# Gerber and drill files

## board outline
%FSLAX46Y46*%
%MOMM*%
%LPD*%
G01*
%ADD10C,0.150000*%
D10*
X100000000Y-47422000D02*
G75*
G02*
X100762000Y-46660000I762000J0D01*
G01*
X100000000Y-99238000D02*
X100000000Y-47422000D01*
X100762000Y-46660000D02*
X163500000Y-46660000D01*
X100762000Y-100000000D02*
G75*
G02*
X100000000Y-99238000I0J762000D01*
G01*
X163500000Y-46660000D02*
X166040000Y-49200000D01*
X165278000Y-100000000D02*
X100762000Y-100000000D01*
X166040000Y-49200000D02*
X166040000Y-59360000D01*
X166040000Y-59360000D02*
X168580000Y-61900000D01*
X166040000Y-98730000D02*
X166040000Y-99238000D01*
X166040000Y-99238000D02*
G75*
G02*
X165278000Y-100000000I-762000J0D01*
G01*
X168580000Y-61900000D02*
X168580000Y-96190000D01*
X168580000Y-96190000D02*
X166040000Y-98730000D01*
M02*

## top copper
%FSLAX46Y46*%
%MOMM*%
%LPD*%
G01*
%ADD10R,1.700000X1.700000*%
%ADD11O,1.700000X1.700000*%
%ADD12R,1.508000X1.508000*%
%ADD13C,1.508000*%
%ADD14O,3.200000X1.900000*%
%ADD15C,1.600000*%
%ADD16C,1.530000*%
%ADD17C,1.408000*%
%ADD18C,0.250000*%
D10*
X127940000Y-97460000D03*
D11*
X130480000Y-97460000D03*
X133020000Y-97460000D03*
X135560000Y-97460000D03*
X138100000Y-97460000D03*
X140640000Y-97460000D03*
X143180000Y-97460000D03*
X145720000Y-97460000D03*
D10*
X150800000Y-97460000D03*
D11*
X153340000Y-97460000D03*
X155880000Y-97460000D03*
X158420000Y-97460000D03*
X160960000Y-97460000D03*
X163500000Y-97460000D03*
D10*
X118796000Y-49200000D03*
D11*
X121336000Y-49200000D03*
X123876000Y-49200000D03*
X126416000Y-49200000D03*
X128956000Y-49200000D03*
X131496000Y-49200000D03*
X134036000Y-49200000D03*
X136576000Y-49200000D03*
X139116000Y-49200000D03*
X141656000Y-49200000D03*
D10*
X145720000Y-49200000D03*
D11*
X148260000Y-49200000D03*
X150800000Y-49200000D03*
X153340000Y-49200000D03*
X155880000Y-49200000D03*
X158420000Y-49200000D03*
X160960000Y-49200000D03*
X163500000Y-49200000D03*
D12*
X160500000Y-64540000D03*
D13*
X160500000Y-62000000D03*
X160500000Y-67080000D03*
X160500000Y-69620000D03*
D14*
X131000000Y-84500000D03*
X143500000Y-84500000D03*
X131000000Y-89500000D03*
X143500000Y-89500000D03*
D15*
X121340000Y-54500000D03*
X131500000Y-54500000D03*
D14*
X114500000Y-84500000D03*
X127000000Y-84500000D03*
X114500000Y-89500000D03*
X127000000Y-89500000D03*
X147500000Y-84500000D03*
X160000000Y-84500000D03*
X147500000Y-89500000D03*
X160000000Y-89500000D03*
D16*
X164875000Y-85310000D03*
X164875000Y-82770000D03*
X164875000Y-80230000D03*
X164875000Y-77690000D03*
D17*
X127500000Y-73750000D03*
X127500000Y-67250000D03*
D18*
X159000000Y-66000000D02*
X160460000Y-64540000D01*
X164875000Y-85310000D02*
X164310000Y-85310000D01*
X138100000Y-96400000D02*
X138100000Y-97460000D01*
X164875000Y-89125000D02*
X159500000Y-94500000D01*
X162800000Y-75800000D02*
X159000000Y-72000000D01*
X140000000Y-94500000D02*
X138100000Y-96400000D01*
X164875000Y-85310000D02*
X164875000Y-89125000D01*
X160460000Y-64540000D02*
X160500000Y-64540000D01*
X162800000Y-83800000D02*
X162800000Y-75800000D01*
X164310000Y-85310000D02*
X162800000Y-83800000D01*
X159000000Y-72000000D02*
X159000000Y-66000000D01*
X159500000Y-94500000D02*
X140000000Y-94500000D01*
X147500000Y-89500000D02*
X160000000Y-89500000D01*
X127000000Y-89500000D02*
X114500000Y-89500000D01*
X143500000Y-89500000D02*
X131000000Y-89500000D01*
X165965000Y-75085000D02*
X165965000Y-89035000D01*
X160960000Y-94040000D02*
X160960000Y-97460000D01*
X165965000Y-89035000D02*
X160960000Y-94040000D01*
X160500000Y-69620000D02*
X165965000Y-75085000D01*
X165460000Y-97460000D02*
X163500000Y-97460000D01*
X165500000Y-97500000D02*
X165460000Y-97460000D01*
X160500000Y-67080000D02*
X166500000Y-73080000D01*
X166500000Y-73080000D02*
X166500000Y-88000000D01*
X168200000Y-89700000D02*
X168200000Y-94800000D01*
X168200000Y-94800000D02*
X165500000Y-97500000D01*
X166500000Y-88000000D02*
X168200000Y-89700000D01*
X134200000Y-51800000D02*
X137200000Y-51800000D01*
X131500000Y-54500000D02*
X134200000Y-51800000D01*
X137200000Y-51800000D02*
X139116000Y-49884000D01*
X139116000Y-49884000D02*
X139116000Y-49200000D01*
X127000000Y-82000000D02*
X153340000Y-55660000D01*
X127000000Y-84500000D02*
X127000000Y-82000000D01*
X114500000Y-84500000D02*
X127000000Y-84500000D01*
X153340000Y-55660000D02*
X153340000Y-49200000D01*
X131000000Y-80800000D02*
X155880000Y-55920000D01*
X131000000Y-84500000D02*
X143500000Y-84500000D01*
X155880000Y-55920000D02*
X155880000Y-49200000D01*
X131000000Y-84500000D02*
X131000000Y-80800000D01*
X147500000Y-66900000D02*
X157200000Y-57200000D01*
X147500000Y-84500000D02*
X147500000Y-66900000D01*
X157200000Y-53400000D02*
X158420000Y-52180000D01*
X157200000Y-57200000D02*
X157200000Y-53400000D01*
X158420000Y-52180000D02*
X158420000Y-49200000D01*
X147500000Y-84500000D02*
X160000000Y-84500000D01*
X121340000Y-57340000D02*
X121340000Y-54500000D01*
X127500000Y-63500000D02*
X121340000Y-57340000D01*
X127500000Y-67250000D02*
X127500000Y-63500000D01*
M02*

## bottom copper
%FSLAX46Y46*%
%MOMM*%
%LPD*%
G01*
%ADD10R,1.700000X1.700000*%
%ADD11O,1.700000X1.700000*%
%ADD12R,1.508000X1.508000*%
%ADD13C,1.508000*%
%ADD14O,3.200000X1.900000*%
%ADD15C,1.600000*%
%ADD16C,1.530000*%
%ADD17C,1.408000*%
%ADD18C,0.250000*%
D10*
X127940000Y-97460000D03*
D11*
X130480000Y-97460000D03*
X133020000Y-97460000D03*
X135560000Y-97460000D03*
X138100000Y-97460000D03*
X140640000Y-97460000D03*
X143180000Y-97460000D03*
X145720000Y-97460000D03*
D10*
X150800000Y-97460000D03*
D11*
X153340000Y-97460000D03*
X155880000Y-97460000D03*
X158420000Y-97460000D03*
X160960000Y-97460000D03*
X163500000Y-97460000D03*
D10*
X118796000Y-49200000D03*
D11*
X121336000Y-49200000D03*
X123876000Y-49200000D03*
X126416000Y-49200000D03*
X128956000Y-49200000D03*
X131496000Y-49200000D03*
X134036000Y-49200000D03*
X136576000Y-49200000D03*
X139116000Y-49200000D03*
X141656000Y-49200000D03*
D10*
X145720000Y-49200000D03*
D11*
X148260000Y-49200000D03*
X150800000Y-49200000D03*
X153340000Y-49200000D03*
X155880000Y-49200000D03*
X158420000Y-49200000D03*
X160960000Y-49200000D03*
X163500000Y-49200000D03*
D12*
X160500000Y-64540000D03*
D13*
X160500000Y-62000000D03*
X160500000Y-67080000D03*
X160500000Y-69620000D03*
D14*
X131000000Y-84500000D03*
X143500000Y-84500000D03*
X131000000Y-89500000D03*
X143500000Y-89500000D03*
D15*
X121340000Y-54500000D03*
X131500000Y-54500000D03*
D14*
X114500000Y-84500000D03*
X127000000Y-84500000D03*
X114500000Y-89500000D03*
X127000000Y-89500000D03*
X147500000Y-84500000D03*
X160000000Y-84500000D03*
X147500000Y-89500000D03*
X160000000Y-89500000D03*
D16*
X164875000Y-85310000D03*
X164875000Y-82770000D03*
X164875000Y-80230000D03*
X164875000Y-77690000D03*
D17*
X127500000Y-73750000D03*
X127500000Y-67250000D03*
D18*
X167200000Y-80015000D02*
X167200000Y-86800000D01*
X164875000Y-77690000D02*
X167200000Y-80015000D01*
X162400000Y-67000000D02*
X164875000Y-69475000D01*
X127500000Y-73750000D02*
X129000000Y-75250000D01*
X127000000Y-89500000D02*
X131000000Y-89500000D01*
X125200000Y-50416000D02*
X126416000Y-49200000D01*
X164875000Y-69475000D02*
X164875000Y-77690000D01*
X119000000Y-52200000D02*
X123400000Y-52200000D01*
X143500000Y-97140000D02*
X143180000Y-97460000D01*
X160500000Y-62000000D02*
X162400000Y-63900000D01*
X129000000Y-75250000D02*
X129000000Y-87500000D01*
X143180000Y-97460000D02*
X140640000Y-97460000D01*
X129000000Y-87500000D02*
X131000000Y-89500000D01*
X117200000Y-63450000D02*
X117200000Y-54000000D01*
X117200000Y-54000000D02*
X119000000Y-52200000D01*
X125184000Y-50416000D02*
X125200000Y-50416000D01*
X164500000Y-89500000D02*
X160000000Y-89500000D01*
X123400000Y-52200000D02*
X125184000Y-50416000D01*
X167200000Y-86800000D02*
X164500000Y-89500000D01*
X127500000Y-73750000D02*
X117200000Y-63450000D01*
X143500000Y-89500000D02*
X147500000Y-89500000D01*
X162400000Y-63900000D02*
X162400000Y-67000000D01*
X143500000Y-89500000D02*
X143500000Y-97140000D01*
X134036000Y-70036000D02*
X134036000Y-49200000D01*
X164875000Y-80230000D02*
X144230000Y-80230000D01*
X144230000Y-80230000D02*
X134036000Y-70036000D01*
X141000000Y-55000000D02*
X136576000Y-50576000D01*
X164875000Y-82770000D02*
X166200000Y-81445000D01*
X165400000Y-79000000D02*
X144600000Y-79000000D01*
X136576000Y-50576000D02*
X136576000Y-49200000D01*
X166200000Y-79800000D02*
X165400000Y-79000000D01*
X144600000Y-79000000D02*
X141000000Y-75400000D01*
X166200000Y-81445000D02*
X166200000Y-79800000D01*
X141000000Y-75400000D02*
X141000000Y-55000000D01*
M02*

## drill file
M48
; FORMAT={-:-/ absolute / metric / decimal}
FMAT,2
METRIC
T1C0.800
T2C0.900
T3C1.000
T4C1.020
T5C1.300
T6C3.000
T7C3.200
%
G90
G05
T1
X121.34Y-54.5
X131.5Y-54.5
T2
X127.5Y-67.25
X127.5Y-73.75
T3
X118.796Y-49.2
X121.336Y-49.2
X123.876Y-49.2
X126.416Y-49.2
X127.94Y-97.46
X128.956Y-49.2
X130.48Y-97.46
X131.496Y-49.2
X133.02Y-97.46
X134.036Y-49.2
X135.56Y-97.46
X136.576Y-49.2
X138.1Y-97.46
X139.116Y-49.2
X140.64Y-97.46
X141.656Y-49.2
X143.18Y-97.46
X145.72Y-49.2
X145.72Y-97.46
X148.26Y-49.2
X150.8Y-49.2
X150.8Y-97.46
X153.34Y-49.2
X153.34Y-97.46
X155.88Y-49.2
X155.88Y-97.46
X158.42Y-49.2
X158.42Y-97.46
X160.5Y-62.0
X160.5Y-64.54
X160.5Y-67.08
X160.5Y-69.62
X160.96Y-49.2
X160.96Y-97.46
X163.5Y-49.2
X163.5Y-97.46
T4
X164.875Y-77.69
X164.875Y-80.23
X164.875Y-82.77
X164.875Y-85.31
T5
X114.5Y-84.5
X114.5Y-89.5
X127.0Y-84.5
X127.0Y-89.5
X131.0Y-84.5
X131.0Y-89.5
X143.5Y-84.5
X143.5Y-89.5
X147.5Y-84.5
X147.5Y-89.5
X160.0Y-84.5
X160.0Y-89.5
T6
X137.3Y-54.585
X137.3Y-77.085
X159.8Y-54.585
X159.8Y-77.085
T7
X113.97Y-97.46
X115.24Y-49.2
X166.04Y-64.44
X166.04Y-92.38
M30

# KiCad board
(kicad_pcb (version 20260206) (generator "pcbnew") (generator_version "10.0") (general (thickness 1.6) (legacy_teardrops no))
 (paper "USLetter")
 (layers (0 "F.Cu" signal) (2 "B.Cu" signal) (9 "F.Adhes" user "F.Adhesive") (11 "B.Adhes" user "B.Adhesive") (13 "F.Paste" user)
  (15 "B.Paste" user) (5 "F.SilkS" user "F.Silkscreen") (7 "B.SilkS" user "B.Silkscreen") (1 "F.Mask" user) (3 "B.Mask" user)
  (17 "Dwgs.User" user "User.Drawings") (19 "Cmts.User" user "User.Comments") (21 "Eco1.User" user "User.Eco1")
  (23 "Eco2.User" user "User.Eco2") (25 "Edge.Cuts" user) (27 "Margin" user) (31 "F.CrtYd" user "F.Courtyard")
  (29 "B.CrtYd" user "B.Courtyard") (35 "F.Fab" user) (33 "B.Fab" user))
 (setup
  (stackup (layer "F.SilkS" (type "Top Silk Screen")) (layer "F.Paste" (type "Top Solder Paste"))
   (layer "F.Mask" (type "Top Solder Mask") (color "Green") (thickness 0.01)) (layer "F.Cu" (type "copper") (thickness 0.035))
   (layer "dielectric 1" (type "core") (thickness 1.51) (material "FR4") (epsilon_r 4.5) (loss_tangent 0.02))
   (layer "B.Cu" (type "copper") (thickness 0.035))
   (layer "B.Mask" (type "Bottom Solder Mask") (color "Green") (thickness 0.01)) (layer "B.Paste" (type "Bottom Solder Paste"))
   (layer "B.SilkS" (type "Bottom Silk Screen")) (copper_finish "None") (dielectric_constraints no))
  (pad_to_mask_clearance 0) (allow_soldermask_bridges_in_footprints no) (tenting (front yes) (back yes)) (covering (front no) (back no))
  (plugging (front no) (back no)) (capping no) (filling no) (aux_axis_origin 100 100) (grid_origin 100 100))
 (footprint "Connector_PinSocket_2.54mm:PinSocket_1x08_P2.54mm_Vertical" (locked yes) (layer "F.Cu") (at 127.94 97.46 90)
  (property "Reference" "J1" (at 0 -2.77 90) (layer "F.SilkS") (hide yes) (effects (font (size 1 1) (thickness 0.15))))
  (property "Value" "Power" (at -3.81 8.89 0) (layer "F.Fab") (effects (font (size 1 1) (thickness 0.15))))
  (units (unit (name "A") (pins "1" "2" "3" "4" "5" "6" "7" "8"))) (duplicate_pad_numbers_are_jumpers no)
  (pad "1" thru_hole rect (at 0 0 90) (size 1.7 1.7) (drill 1) (layers "*.Cu" "*.Mask") (remove_unused_layers no)
   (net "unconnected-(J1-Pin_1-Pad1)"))
  (pad "2" thru_hole oval (at 0 2.54 90) (size 1.7 1.7) (drill 1) (layers "*.Cu" "*.Mask") (remove_unused_layers no) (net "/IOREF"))
  (pad "3" thru_hole oval (at 0 5.08 90) (size 1.7 1.7) (drill 1) (layers "*.Cu" "*.Mask") (remove_unused_layers no) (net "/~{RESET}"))
  (pad "4" thru_hole oval (at 0 7.62 90) (size 1.7 1.7) (drill 1) (layers "*.Cu" "*.Mask") (remove_unused_layers no))
  (pad "5" thru_hole oval (at 0 10.16 90) (size 1.7 1.7) (drill 1) (layers "*.Cu" "*.Mask") (remove_unused_layers no) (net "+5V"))
  (pad "6" thru_hole oval (at 0 12.7 90) (size 1.7 1.7) (drill 1) (layers "*.Cu" "*.Mask") (remove_unused_layers no) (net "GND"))
  (pad "7" thru_hole oval (at 0 15.24 90) (size 1.7 1.7) (drill 1) (layers "*.Cu" "*.Mask") (remove_unused_layers no) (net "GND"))
  (pad "8" thru_hole oval (at 0 17.78 90) (size 1.7 1.7) (drill 1) (layers "*.Cu" "*.Mask") (remove_unused_layers no)
   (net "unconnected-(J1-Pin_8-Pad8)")))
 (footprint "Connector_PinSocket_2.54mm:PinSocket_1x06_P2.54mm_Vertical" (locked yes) (layer "F.Cu") (at 150.8 97.46 90)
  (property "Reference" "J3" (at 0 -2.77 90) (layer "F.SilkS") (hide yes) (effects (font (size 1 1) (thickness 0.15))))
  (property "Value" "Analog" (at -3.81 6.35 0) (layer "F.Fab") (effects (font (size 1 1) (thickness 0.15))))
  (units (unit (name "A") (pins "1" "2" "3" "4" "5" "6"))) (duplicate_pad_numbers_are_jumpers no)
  (pad "1" thru_hole rect (at 0 0 90) (size 1.7 1.7) (drill 1) (layers "*.Cu" "*.Mask") (remove_unused_layers no) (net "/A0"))
  (pad "2" thru_hole oval (at 0 2.54 90) (size 1.7 1.7) (drill 1) (layers "*.Cu" "*.Mask") (remove_unused_layers no) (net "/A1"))
  (pad "3" thru_hole oval (at 0 5.08 90) (size 1.7 1.7) (drill 1) (layers "*.Cu" "*.Mask") (remove_unused_layers no) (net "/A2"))
  (pad "4" thru_hole oval (at 0 7.62 90) (size 1.7 1.7) (drill 1) (layers "*.Cu" "*.Mask") (remove_unused_layers no) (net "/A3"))
  (pad "5" thru_hole oval (at 0 10.16 90) (size 1.7 1.7) (drill 1) (layers "*.Cu" "*.Mask") (remove_unused_layers no) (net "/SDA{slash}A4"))
  (pad "6" thru_hole oval (at 0 12.7 90) (size 1.7 1.7) (drill 1) (layers "*.Cu" "*.Mask") (remove_unused_layers no) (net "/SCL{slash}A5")))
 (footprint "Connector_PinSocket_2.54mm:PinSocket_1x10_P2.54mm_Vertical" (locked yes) (layer "F.Cu") (at 118.796 49.2 90)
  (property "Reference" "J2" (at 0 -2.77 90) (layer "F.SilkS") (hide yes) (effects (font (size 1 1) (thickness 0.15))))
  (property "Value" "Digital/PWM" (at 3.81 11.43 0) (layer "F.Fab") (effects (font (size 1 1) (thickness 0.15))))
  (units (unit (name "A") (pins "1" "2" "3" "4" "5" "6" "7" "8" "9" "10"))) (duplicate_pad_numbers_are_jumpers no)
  (pad "1" thru_hole rect (at 0 0 90) (size 1.7 1.7) (drill 1) (layers "*.Cu" "*.Mask") (remove_unused_layers no))
  (pad "2" thru_hole oval (at 0 2.54 90) (size 1.7 1.7) (drill 1) (layers "*.Cu" "*.Mask") (remove_unused_layers no))
  (pad "3" thru_hole oval (at 0 5.08 90) (size 1.7 1.7) (drill 1) (layers "*.Cu" "*.Mask") (remove_unused_layers no) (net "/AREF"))
  (pad "4" thru_hole oval (at 0 7.62 90) (size 1.7 1.7) (drill 1) (layers "*.Cu" "*.Mask") (remove_unused_layers no) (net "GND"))
  (pad "5" thru_hole oval (at 0 10.16 90) (size 1.7 1.7) (drill 1) (layers "*.Cu" "*.Mask") (remove_unused_layers no) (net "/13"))
  (pad "6" thru_hole oval (at 0 12.7 90) (size 1.7 1.7) (drill 1) (layers "*.Cu" "*.Mask") (remove_unused_layers no) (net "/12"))
  (pad "7" thru_hole oval (at 0 15.24 90) (size 1.7 1.7) (drill 1) (layers "*.Cu" "*.Mask") (remove_unused_layers no) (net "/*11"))
  (pad "8" thru_hole oval (at 0 17.78 90) (size 1.7 1.7) (drill 1) (layers "*.Cu" "*.Mask") (remove_unused_layers no) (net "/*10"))
  (pad "9" thru_hole oval (at 0 20.32 90) (size 1.7 1.7) (drill 1) (layers "*.Cu" "*.Mask") (remove_unused_layers no) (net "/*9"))
  (pad "10" thru_hole oval (at 0 22.86 90) (size 1.7 1.7) (drill 1) (layers "*.Cu" "*.Mask") (remove_unused_layers no) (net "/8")))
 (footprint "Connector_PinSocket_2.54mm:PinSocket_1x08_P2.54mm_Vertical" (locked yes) (layer "F.Cu") (at 145.72 49.2 90)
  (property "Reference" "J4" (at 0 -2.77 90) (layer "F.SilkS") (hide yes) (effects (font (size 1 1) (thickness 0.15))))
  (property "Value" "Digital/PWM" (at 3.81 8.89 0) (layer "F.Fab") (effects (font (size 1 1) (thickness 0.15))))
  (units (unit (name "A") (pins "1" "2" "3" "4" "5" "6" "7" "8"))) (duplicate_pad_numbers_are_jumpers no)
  (pad "1" thru_hole rect (at 0 0 90) (size 1.7 1.7) (drill 1) (layers "*.Cu" "*.Mask") (remove_unused_layers no) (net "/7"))
  (pad "2" thru_hole oval (at 0 2.54 90) (size 1.7 1.7) (drill 1) (layers "*.Cu" "*.Mask") (remove_unused_layers no) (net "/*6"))
  (pad "3" thru_hole oval (at 0 5.08 90) (size 1.7 1.7) (drill 1) (layers "*.Cu" "*.Mask") (remove_unused_layers no) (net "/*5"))
  (pad "4" thru_hole oval (at 0 7.62 90) (size 1.7 1.7) (drill 1) (layers "*.Cu" "*.Mask") (remove_unused_layers no) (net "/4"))
  (pad "5" thru_hole oval (at 0 10.16 90) (size 1.7 1.7) (drill 1) (layers "*.Cu" "*.Mask") (remove_unused_layers no) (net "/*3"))
  (pad "6" thru_hole oval (at 0 12.7 90) (size 1.7 1.7) (drill 1) (layers "*.Cu" "*.Mask") (remove_unused_layers no) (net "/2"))
  (pad "7" thru_hole oval (at 0 15.24 90) (size 1.7 1.7) (drill 1) (layers "*.Cu" "*.Mask") (remove_unused_layers no) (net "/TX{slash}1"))
  (pad "8" thru_hole oval (at 0 17.78 90) (size 1.7 1.7) (drill 1) (layers "*.Cu" "*.Mask") (remove_unused_layers no) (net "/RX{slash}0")))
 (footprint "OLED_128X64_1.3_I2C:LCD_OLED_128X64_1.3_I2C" (layer "F.Cu") (at 148.55 65.81 -90)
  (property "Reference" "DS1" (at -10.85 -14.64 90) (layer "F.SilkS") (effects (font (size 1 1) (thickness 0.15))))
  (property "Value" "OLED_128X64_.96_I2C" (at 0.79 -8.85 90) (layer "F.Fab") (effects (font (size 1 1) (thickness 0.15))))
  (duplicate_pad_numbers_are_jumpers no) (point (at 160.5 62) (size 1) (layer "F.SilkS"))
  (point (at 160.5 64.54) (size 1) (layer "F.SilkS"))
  (pad "" np_thru_hole circle (at -11.225 -11.25 270) (size 3 3) (drill 3) (layers "*.Cu" "*.Mask"))
  (pad "" np_thru_hole circle (at -11.225 11.25 270) (size 3 3) (drill 3) (layers "*.Cu" "*.Mask"))
  (pad "" np_thru_hole circle (at 11.275 -11.25 270) (size 3 3) (drill 3) (layers "*.Cu" "*.Mask"))
  (pad "" np_thru_hole circle (at 11.275 11.25 270) (size 3 3) (drill 3) (layers "*.Cu" "*.Mask"))
  (pad "1" thru_hole rect (at -1.27 -11.95 270) (size 1.508 1.508) (drill 1) (layers "*.Cu" "*.Mask") (remove_unused_layers no) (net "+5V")
   (solder_mask_margin 0.102))
  (pad "2" thru_hole circle (at -3.81 -11.95 270) (size 1.508 1.508) (drill 1) (layers "*.Cu" "*.Mask") (remove_unused_layers no)
   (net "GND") (solder_mask_margin 0.102))
  (pad "3" thru_hole circle (at 1.27 -11.95 270) (size 1.508 1.508) (drill 1) (layers "*.Cu" "*.Mask") (remove_unused_layers no)
   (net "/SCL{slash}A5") (solder_mask_margin 0.102))
  (pad "4" thru_hole circle (at 3.81 -11.95 270) (size 1.508 1.508) (drill 1) (layers "*.Cu" "*.Mask") (remove_unused_layers no)
   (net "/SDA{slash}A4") (solder_mask_margin 0.102)))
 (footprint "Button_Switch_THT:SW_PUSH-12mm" (layer "F.Cu") (at 131 84.5)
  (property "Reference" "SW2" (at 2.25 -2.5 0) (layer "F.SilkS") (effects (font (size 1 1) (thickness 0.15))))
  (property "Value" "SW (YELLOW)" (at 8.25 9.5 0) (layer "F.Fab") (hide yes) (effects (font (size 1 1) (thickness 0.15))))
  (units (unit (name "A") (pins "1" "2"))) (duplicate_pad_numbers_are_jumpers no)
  (pad "1" thru_hole oval (at 0 0) (size 3.2 1.9) (drill 1.3) (layers "*.Cu" "*.Mask") (remove_unused_layers no) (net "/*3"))
  (pad "1" thru_hole oval (at 12.5 0) (size 3.2 1.9) (drill 1.3) (layers "*.Cu" "*.Mask") (remove_unused_layers no) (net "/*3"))
  (pad "2" thru_hole oval (at 0 5) (size 3.2 1.9) (drill 1.3) (layers "*.Cu" "*.Mask") (remove_unused_layers no) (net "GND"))
  (pad "2" thru_hole oval (at 12.5 5) (size 3.2 1.9) (drill 1.3) (layers "*.Cu" "*.Mask") (remove_unused_layers no) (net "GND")))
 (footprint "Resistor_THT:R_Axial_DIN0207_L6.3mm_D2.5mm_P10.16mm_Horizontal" (layer "F.Cu") (at 121.34 54.5)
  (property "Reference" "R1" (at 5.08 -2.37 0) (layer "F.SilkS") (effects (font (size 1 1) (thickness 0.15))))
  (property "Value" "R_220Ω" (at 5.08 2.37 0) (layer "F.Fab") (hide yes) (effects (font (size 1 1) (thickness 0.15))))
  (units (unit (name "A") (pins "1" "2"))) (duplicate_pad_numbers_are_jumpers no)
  (pad "1" thru_hole circle (at 0 0) (size 1.6 1.6) (drill 0.8) (layers "*.Cu" "*.Mask") (remove_unused_layers no) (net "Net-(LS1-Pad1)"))
  (pad "2" thru_hole circle (at 10.16 0) (size 1.6 1.6) (drill 0.8) (layers "*.Cu" "*.Mask") (remove_unused_layers no) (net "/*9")))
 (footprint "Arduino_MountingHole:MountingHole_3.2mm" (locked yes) (layer "F.Cu") (at 115.24 49.2)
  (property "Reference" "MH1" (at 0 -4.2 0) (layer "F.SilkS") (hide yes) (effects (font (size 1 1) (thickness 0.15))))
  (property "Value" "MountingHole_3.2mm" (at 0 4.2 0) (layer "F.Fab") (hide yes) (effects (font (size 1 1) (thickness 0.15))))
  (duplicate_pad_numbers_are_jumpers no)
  (pad "" np_thru_hole circle (at 0 0) (size 3.2 3.2) (drill 3.2) (layers "*.Cu" "*.Mask")))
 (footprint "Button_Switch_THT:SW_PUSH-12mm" (layer "F.Cu") (at 114.5 84.5)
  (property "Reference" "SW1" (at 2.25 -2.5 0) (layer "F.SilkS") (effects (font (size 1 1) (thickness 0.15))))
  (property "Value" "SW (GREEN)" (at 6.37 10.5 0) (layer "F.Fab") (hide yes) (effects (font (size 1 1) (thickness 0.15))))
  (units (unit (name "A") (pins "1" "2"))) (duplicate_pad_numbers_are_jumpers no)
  (pad "1" thru_hole oval (at 0 0) (size 3.2 1.9) (drill 1.3) (layers "*.Cu" "*.Mask") (remove_unused_layers no) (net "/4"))
  (pad "1" thru_hole oval (at 12.5 0) (size 3.2 1.9) (drill 1.3) (layers "*.Cu" "*.Mask") (remove_unused_layers no) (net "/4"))
  (pad "2" thru_hole oval (at 0 5) (size 3.2 1.9) (drill 1.3) (layers "*.Cu" "*.Mask") (remove_unused_layers no) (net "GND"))
  (pad "2" thru_hole oval (at 12.5 5) (size 3.2 1.9) (drill 1.3) (layers "*.Cu" "*.Mask") (remove_unused_layers no) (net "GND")))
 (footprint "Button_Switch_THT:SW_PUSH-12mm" (layer "F.Cu") (at 147.5 84.5)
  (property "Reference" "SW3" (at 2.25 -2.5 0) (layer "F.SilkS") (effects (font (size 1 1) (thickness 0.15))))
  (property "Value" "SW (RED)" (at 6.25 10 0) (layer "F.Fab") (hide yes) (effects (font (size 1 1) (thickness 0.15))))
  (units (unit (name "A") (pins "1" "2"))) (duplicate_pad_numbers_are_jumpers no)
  (pad "1" thru_hole oval (at 0 0) (size 3.2 1.9) (drill 1.3) (layers "*.Cu" "*.Mask") (remove_unused_layers no) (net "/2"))
  (pad "1" thru_hole oval (at 12.5 0) (size 3.2 1.9) (drill 1.3) (layers "*.Cu" "*.Mask") (remove_unused_layers no) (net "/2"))
  (pad "2" thru_hole oval (at 0 5) (size 3.2 1.9) (drill 1.3) (layers "*.Cu" "*.Mask") (remove_unused_layers no) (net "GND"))
  (pad "2" thru_hole oval (at 12.5 5) (size 3.2 1.9) (drill 1.3) (layers "*.Cu" "*.Mask") (remove_unused_layers no) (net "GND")))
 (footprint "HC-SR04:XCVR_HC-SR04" (layer "F.Cu") (at 164.875 81.5 90)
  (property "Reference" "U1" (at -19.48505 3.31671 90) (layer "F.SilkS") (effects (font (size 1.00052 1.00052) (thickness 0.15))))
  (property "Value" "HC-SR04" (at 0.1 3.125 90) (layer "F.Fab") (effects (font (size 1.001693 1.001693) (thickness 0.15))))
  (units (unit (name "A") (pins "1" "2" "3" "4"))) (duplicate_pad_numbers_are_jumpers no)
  (pad "1" thru_hole circle (at -3.81 0 90) (size 1.53 1.53) (drill 1.02) (layers "*.Cu" "*.Mask") (remove_unused_layers no) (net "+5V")
   (solder_mask_margin 0.102))
  (pad "2" thru_hole circle (at -1.27 0 90) (size 1.53 1.53) (drill 1.02) (layers "*.Cu" "*.Mask") (remove_unused_layers no) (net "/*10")
   (solder_mask_margin 0.102))
  (pad "3" thru_hole circle (at 1.27 0 90) (size 1.53 1.53) (drill 1.02) (layers "*.Cu" "*.Mask") (remove_unused_layers no) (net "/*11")
   (solder_mask_margin 0.102))
  (pad "4" thru_hole circle (at 3.81 0 90) (size 1.53 1.53) (drill 1.02) (layers "*.Cu" "*.Mask") (remove_unused_layers no) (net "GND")
   (solder_mask_margin 0.102)))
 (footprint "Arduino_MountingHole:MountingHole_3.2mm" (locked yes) (layer "F.Cu") (at 113.97 97.46)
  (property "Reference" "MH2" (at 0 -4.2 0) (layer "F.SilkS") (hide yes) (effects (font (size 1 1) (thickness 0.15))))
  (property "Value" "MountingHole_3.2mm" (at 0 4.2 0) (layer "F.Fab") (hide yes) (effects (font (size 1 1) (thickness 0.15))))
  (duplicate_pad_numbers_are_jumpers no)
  (pad "" np_thru_hole circle (at 0 0) (size 3.2 3.2) (drill 3.2) (layers "*.Cu" "*.Mask")))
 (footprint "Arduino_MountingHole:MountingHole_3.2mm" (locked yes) (layer "F.Cu") (at 166.04 64.44)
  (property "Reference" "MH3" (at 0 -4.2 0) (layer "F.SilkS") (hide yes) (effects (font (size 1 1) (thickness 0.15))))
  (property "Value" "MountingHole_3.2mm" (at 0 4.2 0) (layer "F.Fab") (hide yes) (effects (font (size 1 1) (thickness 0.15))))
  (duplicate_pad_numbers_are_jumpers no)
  (pad "" np_thru_hole circle (at 0 0) (size 3.2 3.2) (drill 3.2) (layers "*.Cu" "*.Mask")))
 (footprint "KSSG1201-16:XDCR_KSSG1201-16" (layer "F.Cu") (at 127.5 70.5 -90)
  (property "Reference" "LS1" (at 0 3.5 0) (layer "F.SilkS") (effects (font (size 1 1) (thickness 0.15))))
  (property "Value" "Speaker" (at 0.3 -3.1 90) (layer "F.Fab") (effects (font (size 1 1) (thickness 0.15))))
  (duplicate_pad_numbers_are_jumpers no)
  (pad "N" thru_hole circle (at 3.25 0 270) (size 1.408 1.408) (drill 0.9) (layers "*.Cu" "*.Mask") (remove_unused_layers no) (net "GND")
   (solder_mask_margin 0.102))
  (pad "P" thru_hole circle (at -3.25 0 270) (size 1.408 1.408) (drill 0.9) (layers "*.Cu" "*.Mask") (remove_unused_layers no)
   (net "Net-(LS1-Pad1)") (solder_mask_margin 0.102)))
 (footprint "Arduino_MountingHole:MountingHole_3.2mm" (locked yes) (layer "F.Cu") (at 166.04 92.38)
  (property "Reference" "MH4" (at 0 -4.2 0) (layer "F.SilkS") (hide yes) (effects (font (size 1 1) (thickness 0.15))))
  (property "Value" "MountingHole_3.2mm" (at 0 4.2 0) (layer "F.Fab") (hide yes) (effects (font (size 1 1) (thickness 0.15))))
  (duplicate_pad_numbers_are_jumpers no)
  (pad "" np_thru_hole circle (at 0 0) (size 3.2 3.2) (drill 3.2) (layers "*.Cu" "*.Mask")))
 (gr_arc (start 100 47.422) (mid 100.223185 46.883185) (end 100.762 46.66) (stroke (width 0.15) (type solid)) (layer "Edge.Cuts"))
 (gr_line (start 100 99.238) (end 100 47.422) (stroke (width 0.15) (type solid)) (layer "Edge.Cuts"))
 (gr_line (start 100.762 46.66) (end 163.5 46.66) (stroke (width 0.15) (type solid)) (layer "Edge.Cuts"))
 (gr_arc (start 100.762 100) (mid 100.223185 99.776815) (end 100 99.238) (stroke (width 0.15) (type solid)) (layer "Edge.Cuts"))
 (gr_line (start 163.5 46.66) (end 166.04 49.2) (stroke (width 0.15) (type solid)) (layer "Edge.Cuts"))
 (gr_line (start 165.278 100) (end 100.762 100) (stroke (width 0.15) (type solid)) (layer "Edge.Cuts"))
 (gr_line (start 166.04 49.2) (end 166.04 59.36) (stroke (width 0.15) (type solid)) (layer "Edge.Cuts"))
 (gr_line (start 166.04 59.36) (end 168.58 61.9) (stroke (width 0.15) (type solid)) (layer "Edge.Cuts"))
 (gr_line (start 166.04 98.73) (end 166.04 99.238) (stroke (width 0.15) (type solid)) (layer "Edge.Cuts"))
 (gr_arc (start 166.04 99.238) (mid 165.816815 99.776815) (end 165.278 100) (stroke (width 0.15) (type solid)) (layer "Edge.Cuts"))
 (gr_line (start 168.58 61.9) (end 168.58 96.19) (stroke (width 0.15) (type solid)) (layer "Edge.Cuts"))
 (gr_line (start 168.58 96.19) (end 166.04 98.73) (stroke (width 0.15) (type solid)) (layer "Edge.Cuts"))
 (segment (start 159 66) (end 160.46 64.54) (width 0.25) (layer "F.Cu") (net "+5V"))
 (segment (start 164.875 85.31) (end 164.31 85.31) (width 0.25) (layer "F.Cu") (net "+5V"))
 (segment (start 138.1 96.4) (end 138.1 97.46) (width 0.25) (layer "F.Cu") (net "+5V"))
 (segment (start 164.875 89.125) (end 159.5 94.5) (width 0.25) (layer "F.Cu") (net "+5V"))
 (segment (start 162.8 75.8) (end 159 72) (width 0.25) (layer "F.Cu") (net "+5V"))
 (segment (start 140 94.5) (end 138.1 96.4) (width 0.25) (layer "F.Cu") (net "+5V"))
 (segment (start 164.875 85.31) (end 164.875 89.125) (width 0.25) (layer "F.Cu") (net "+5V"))
 (segment (start 160.46 64.54) (end 160.5 64.54) (width 0.25) (layer "F.Cu") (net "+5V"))
 (segment (start 162.8 83.8) (end 162.8 75.8) (width 0.25) (layer "F.Cu") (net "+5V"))
 (segment (start 164.31 85.31) (end 162.8 83.8) (width 0.25) (layer "F.Cu") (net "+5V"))
 (segment (start 159 72) (end 159 66) (width 0.25) (layer "F.Cu") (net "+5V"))
 (segment (start 159.5 94.5) (end 140 94.5) (width 0.25) (layer "F.Cu") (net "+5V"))
 (segment (start 147.5 89.5) (end 160 89.5) (width 0.25) (layer "F.Cu") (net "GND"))
 (segment (start 127 89.5) (end 114.5 89.5) (width 0.25) (layer "F.Cu") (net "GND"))
 (segment (start 143.5 89.5) (end 131 89.5) (width 0.25) (layer "F.Cu") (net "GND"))
 (segment (start 167.2 80.015) (end 167.2 86.8) (width 0.25) (layer "B.Cu") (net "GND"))
 (segment (start 164.875 77.69) (end 167.2 80.015) (width 0.25) (layer "B.Cu") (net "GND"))
 (segment (start 162.4 67) (end 164.875 69.475) (width 0.25) (layer "B.Cu") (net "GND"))
 (segment (start 127.5 73.75) (end 129 75.25) (width 0.25) (layer "B.Cu") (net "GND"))
 (segment (start 127 89.5) (end 131 89.5) (width 0.25) (layer "B.Cu") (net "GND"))
 (segment (start 125.2 50.416) (end 126.416 49.2) (width 0.25) (layer "B.Cu") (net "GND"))
 (segment (start 164.875 69.475) (end 164.875 77.69) (width 0.25) (layer "B.Cu") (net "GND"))
 (segment (start 119 52.2) (end 123.4 52.2) (width 0.25) (layer "B.Cu") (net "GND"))
 (segment (start 143.5 97.14) (end 143.18 97.46) (width 0.25) (layer "B.Cu") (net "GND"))
 (segment (start 160.5 62) (end 162.4 63.9) (width 0.25) (layer "B.Cu") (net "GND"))
 (segment (start 129 75.25) (end 129 87.5) (width 0.25) (layer "B.Cu") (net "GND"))
 (segment (start 143.18 97.46) (end 140.64 97.46) (width 0.25) (layer "B.Cu") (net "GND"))
 (segment (start 129 87.5) (end 131 89.5) (width 0.25) (layer "B.Cu") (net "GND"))
 (segment (start 117.2 63.45) (end 117.2 54) (width 0.25) (layer "B.Cu") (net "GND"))
 (segment (start 117.2 54) (end 119 52.2) (width 0.25) (layer "B.Cu") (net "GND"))
 (segment (start 125.184 50.416) (end 125.2 50.416) (width 0.25) (layer "B.Cu") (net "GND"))
 (segment (start 164.5 89.5) (end 160 89.5) (width 0.25) (layer "B.Cu") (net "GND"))
 (segment (start 123.4 52.2) (end 125.184 50.416) (width 0.25) (layer "B.Cu") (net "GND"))
 (segment (start 167.2 86.8) (end 164.5 89.5) (width 0.25) (layer "B.Cu") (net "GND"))
 (segment (start 127.5 73.75) (end 117.2 63.45) (width 0.25) (layer "B.Cu") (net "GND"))
 (segment (start 143.5 89.5) (end 147.5 89.5) (width 0.25) (layer "B.Cu") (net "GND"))
 (segment (start 162.4 63.9) (end 162.4 67) (width 0.25) (layer "B.Cu") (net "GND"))
 (segment (start 143.5 89.5) (end 143.5 97.14) (width 0.25) (layer "B.Cu") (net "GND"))
 (segment (start 165.965 75.085) (end 165.965 89.035) (width 0.25) (layer "F.Cu") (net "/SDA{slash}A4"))
 (segment (start 160.96 94.04) (end 160.96 97.46) (width 0.25) (layer "F.Cu") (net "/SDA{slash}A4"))
 (segment (start 165.965 89.035) (end 160.96 94.04) (width 0.25) (layer "F.Cu") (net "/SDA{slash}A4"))
 (segment (start 160.5 69.62) (end 165.965 75.085) (width 0.25) (layer "F.Cu") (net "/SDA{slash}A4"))
 (segment (start 165.46 97.46) (end 163.5 97.46) (width 0.25) (layer "F.Cu") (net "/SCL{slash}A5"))
 (segment (start 165.5 97.5) (end 165.46 97.46) (width 0.25) (layer "F.Cu") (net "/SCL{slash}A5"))
 (segment (start 160.5 67.08) (end 166.5 73.08) (width 0.25) (layer "F.Cu") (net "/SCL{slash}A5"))
 (segment (start 166.5 73.08) (end 166.5 88) (width 0.25) (layer "F.Cu") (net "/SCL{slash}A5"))
 (segment (start 168.2 89.7) (end 168.2 94.8) (width 0.25) (layer "F.Cu") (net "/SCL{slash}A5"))
 (segment (start 168.2 94.8) (end 165.5 97.5) (width 0.25) (layer "F.Cu") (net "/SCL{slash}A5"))
 (segment (start 166.5 88) (end 168.2 89.7) (width 0.25) (layer "F.Cu") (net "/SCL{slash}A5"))
 (segment (start 134.036 70.036) (end 134.036 49.2) (width 0.25) (layer "B.Cu") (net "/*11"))
 (segment (start 164.875 80.23) (end 144.23 80.23) (width 0.25) (layer "B.Cu") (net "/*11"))
 (segment (start 144.23 80.23) (end 134.036 70.036) (width 0.25) (layer "B.Cu") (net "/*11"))
 (segment (start 141 55) (end 136.576 50.576) (width 0.25) (layer "B.Cu") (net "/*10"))
 (segment (start 164.875 82.77) (end 166.2 81.445) (width 0.25) (layer "B.Cu") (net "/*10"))
 (segment (start 165.4 79) (end 144.6 79) (width 0.25) (layer "B.Cu") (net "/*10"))
 (segment (start 136.576 50.576) (end 136.576 49.2) (width 0.25) (layer "B.Cu") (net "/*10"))
 (segment (start 166.2 79.8) (end 165.4 79) (width 0.25) (layer "B.Cu") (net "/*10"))
 (segment (start 144.6 79) (end 141 75.4) (width 0.25) (layer "B.Cu") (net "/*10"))
 (segment (start 166.2 81.445) (end 166.2 79.8) (width 0.25) (layer "B.Cu") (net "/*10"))
 (segment (start 141 75.4) (end 141 55) (width 0.25) (layer "B.Cu") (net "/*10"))
 (segment (start 134.2 51.8) (end 137.2 51.8) (width 0.25) (layer "F.Cu") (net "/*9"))
 (segment (start 131.5 54.5) (end 134.2 51.8) (width 0.25) (layer "F.Cu") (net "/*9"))
 (segment (start 137.2 51.8) (end 139.116 49.884) (width 0.25) (layer "F.Cu") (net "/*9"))
 (segment (start 139.116 49.884) (end 139.116 49.2) (width 0.25) (layer "F.Cu") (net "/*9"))
 (segment (start 127 82) (end 153.34 55.66) (width 0.25) (layer "F.Cu") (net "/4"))
 (segment (start 127 84.5) (end 127 82) (width 0.25) (layer "F.Cu") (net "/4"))
 (segment (start 114.5 84.5) (end 127 84.5) (width 0.25) (layer "F.Cu") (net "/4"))
 (segment (start 153.34 55.66) (end 153.34 49.2) (width 0.25) (layer "F.Cu") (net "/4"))
 (segment (start 131 80.8) (end 155.88 55.92) (width 0.25) (layer "F.Cu") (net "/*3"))
 (segment (start 131 84.5) (end 143.5 84.5) (width 0.25) (layer "F.Cu") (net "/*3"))
 (segment (start 155.88 55.92) (end 155.88 49.2) (width 0.25) (layer "F.Cu") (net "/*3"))
 (segment (start 131 84.5) (end 131 80.8) (width 0.25) (layer "F.Cu") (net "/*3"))
 (segment (start 147.5 66.9) (end 157.2 57.2) (width 0.25) (layer "F.Cu") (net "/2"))
 (segment (start 147.5 84.5) (end 147.5 66.9) (width 0.25) (layer "F.Cu") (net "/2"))
 (segment (start 157.2 53.4) (end 158.42 52.18) (width 0.25) (layer "F.Cu") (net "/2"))
 (segment (start 157.2 57.2) (end 157.2 53.4) (width 0.25) (layer "F.Cu") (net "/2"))
 (segment (start 158.42 52.18) (end 158.42 49.2) (width 0.25) (layer "F.Cu") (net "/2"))
 (segment (start 147.5 84.5) (end 160 84.5) (width 0.25) (layer "F.Cu") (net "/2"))
 (segment (start 121.34 57.34) (end 121.34 54.5) (width 0.25) (layer "F.Cu") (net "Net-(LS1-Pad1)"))
 (segment (start 127.5 63.5) (end 121.34 57.34) (width 0.25) (layer "F.Cu") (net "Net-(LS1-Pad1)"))
 (segment (start 127.5 67.25) (end 127.5 63.5) (width 0.25) (layer "F.Cu") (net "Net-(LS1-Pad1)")))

